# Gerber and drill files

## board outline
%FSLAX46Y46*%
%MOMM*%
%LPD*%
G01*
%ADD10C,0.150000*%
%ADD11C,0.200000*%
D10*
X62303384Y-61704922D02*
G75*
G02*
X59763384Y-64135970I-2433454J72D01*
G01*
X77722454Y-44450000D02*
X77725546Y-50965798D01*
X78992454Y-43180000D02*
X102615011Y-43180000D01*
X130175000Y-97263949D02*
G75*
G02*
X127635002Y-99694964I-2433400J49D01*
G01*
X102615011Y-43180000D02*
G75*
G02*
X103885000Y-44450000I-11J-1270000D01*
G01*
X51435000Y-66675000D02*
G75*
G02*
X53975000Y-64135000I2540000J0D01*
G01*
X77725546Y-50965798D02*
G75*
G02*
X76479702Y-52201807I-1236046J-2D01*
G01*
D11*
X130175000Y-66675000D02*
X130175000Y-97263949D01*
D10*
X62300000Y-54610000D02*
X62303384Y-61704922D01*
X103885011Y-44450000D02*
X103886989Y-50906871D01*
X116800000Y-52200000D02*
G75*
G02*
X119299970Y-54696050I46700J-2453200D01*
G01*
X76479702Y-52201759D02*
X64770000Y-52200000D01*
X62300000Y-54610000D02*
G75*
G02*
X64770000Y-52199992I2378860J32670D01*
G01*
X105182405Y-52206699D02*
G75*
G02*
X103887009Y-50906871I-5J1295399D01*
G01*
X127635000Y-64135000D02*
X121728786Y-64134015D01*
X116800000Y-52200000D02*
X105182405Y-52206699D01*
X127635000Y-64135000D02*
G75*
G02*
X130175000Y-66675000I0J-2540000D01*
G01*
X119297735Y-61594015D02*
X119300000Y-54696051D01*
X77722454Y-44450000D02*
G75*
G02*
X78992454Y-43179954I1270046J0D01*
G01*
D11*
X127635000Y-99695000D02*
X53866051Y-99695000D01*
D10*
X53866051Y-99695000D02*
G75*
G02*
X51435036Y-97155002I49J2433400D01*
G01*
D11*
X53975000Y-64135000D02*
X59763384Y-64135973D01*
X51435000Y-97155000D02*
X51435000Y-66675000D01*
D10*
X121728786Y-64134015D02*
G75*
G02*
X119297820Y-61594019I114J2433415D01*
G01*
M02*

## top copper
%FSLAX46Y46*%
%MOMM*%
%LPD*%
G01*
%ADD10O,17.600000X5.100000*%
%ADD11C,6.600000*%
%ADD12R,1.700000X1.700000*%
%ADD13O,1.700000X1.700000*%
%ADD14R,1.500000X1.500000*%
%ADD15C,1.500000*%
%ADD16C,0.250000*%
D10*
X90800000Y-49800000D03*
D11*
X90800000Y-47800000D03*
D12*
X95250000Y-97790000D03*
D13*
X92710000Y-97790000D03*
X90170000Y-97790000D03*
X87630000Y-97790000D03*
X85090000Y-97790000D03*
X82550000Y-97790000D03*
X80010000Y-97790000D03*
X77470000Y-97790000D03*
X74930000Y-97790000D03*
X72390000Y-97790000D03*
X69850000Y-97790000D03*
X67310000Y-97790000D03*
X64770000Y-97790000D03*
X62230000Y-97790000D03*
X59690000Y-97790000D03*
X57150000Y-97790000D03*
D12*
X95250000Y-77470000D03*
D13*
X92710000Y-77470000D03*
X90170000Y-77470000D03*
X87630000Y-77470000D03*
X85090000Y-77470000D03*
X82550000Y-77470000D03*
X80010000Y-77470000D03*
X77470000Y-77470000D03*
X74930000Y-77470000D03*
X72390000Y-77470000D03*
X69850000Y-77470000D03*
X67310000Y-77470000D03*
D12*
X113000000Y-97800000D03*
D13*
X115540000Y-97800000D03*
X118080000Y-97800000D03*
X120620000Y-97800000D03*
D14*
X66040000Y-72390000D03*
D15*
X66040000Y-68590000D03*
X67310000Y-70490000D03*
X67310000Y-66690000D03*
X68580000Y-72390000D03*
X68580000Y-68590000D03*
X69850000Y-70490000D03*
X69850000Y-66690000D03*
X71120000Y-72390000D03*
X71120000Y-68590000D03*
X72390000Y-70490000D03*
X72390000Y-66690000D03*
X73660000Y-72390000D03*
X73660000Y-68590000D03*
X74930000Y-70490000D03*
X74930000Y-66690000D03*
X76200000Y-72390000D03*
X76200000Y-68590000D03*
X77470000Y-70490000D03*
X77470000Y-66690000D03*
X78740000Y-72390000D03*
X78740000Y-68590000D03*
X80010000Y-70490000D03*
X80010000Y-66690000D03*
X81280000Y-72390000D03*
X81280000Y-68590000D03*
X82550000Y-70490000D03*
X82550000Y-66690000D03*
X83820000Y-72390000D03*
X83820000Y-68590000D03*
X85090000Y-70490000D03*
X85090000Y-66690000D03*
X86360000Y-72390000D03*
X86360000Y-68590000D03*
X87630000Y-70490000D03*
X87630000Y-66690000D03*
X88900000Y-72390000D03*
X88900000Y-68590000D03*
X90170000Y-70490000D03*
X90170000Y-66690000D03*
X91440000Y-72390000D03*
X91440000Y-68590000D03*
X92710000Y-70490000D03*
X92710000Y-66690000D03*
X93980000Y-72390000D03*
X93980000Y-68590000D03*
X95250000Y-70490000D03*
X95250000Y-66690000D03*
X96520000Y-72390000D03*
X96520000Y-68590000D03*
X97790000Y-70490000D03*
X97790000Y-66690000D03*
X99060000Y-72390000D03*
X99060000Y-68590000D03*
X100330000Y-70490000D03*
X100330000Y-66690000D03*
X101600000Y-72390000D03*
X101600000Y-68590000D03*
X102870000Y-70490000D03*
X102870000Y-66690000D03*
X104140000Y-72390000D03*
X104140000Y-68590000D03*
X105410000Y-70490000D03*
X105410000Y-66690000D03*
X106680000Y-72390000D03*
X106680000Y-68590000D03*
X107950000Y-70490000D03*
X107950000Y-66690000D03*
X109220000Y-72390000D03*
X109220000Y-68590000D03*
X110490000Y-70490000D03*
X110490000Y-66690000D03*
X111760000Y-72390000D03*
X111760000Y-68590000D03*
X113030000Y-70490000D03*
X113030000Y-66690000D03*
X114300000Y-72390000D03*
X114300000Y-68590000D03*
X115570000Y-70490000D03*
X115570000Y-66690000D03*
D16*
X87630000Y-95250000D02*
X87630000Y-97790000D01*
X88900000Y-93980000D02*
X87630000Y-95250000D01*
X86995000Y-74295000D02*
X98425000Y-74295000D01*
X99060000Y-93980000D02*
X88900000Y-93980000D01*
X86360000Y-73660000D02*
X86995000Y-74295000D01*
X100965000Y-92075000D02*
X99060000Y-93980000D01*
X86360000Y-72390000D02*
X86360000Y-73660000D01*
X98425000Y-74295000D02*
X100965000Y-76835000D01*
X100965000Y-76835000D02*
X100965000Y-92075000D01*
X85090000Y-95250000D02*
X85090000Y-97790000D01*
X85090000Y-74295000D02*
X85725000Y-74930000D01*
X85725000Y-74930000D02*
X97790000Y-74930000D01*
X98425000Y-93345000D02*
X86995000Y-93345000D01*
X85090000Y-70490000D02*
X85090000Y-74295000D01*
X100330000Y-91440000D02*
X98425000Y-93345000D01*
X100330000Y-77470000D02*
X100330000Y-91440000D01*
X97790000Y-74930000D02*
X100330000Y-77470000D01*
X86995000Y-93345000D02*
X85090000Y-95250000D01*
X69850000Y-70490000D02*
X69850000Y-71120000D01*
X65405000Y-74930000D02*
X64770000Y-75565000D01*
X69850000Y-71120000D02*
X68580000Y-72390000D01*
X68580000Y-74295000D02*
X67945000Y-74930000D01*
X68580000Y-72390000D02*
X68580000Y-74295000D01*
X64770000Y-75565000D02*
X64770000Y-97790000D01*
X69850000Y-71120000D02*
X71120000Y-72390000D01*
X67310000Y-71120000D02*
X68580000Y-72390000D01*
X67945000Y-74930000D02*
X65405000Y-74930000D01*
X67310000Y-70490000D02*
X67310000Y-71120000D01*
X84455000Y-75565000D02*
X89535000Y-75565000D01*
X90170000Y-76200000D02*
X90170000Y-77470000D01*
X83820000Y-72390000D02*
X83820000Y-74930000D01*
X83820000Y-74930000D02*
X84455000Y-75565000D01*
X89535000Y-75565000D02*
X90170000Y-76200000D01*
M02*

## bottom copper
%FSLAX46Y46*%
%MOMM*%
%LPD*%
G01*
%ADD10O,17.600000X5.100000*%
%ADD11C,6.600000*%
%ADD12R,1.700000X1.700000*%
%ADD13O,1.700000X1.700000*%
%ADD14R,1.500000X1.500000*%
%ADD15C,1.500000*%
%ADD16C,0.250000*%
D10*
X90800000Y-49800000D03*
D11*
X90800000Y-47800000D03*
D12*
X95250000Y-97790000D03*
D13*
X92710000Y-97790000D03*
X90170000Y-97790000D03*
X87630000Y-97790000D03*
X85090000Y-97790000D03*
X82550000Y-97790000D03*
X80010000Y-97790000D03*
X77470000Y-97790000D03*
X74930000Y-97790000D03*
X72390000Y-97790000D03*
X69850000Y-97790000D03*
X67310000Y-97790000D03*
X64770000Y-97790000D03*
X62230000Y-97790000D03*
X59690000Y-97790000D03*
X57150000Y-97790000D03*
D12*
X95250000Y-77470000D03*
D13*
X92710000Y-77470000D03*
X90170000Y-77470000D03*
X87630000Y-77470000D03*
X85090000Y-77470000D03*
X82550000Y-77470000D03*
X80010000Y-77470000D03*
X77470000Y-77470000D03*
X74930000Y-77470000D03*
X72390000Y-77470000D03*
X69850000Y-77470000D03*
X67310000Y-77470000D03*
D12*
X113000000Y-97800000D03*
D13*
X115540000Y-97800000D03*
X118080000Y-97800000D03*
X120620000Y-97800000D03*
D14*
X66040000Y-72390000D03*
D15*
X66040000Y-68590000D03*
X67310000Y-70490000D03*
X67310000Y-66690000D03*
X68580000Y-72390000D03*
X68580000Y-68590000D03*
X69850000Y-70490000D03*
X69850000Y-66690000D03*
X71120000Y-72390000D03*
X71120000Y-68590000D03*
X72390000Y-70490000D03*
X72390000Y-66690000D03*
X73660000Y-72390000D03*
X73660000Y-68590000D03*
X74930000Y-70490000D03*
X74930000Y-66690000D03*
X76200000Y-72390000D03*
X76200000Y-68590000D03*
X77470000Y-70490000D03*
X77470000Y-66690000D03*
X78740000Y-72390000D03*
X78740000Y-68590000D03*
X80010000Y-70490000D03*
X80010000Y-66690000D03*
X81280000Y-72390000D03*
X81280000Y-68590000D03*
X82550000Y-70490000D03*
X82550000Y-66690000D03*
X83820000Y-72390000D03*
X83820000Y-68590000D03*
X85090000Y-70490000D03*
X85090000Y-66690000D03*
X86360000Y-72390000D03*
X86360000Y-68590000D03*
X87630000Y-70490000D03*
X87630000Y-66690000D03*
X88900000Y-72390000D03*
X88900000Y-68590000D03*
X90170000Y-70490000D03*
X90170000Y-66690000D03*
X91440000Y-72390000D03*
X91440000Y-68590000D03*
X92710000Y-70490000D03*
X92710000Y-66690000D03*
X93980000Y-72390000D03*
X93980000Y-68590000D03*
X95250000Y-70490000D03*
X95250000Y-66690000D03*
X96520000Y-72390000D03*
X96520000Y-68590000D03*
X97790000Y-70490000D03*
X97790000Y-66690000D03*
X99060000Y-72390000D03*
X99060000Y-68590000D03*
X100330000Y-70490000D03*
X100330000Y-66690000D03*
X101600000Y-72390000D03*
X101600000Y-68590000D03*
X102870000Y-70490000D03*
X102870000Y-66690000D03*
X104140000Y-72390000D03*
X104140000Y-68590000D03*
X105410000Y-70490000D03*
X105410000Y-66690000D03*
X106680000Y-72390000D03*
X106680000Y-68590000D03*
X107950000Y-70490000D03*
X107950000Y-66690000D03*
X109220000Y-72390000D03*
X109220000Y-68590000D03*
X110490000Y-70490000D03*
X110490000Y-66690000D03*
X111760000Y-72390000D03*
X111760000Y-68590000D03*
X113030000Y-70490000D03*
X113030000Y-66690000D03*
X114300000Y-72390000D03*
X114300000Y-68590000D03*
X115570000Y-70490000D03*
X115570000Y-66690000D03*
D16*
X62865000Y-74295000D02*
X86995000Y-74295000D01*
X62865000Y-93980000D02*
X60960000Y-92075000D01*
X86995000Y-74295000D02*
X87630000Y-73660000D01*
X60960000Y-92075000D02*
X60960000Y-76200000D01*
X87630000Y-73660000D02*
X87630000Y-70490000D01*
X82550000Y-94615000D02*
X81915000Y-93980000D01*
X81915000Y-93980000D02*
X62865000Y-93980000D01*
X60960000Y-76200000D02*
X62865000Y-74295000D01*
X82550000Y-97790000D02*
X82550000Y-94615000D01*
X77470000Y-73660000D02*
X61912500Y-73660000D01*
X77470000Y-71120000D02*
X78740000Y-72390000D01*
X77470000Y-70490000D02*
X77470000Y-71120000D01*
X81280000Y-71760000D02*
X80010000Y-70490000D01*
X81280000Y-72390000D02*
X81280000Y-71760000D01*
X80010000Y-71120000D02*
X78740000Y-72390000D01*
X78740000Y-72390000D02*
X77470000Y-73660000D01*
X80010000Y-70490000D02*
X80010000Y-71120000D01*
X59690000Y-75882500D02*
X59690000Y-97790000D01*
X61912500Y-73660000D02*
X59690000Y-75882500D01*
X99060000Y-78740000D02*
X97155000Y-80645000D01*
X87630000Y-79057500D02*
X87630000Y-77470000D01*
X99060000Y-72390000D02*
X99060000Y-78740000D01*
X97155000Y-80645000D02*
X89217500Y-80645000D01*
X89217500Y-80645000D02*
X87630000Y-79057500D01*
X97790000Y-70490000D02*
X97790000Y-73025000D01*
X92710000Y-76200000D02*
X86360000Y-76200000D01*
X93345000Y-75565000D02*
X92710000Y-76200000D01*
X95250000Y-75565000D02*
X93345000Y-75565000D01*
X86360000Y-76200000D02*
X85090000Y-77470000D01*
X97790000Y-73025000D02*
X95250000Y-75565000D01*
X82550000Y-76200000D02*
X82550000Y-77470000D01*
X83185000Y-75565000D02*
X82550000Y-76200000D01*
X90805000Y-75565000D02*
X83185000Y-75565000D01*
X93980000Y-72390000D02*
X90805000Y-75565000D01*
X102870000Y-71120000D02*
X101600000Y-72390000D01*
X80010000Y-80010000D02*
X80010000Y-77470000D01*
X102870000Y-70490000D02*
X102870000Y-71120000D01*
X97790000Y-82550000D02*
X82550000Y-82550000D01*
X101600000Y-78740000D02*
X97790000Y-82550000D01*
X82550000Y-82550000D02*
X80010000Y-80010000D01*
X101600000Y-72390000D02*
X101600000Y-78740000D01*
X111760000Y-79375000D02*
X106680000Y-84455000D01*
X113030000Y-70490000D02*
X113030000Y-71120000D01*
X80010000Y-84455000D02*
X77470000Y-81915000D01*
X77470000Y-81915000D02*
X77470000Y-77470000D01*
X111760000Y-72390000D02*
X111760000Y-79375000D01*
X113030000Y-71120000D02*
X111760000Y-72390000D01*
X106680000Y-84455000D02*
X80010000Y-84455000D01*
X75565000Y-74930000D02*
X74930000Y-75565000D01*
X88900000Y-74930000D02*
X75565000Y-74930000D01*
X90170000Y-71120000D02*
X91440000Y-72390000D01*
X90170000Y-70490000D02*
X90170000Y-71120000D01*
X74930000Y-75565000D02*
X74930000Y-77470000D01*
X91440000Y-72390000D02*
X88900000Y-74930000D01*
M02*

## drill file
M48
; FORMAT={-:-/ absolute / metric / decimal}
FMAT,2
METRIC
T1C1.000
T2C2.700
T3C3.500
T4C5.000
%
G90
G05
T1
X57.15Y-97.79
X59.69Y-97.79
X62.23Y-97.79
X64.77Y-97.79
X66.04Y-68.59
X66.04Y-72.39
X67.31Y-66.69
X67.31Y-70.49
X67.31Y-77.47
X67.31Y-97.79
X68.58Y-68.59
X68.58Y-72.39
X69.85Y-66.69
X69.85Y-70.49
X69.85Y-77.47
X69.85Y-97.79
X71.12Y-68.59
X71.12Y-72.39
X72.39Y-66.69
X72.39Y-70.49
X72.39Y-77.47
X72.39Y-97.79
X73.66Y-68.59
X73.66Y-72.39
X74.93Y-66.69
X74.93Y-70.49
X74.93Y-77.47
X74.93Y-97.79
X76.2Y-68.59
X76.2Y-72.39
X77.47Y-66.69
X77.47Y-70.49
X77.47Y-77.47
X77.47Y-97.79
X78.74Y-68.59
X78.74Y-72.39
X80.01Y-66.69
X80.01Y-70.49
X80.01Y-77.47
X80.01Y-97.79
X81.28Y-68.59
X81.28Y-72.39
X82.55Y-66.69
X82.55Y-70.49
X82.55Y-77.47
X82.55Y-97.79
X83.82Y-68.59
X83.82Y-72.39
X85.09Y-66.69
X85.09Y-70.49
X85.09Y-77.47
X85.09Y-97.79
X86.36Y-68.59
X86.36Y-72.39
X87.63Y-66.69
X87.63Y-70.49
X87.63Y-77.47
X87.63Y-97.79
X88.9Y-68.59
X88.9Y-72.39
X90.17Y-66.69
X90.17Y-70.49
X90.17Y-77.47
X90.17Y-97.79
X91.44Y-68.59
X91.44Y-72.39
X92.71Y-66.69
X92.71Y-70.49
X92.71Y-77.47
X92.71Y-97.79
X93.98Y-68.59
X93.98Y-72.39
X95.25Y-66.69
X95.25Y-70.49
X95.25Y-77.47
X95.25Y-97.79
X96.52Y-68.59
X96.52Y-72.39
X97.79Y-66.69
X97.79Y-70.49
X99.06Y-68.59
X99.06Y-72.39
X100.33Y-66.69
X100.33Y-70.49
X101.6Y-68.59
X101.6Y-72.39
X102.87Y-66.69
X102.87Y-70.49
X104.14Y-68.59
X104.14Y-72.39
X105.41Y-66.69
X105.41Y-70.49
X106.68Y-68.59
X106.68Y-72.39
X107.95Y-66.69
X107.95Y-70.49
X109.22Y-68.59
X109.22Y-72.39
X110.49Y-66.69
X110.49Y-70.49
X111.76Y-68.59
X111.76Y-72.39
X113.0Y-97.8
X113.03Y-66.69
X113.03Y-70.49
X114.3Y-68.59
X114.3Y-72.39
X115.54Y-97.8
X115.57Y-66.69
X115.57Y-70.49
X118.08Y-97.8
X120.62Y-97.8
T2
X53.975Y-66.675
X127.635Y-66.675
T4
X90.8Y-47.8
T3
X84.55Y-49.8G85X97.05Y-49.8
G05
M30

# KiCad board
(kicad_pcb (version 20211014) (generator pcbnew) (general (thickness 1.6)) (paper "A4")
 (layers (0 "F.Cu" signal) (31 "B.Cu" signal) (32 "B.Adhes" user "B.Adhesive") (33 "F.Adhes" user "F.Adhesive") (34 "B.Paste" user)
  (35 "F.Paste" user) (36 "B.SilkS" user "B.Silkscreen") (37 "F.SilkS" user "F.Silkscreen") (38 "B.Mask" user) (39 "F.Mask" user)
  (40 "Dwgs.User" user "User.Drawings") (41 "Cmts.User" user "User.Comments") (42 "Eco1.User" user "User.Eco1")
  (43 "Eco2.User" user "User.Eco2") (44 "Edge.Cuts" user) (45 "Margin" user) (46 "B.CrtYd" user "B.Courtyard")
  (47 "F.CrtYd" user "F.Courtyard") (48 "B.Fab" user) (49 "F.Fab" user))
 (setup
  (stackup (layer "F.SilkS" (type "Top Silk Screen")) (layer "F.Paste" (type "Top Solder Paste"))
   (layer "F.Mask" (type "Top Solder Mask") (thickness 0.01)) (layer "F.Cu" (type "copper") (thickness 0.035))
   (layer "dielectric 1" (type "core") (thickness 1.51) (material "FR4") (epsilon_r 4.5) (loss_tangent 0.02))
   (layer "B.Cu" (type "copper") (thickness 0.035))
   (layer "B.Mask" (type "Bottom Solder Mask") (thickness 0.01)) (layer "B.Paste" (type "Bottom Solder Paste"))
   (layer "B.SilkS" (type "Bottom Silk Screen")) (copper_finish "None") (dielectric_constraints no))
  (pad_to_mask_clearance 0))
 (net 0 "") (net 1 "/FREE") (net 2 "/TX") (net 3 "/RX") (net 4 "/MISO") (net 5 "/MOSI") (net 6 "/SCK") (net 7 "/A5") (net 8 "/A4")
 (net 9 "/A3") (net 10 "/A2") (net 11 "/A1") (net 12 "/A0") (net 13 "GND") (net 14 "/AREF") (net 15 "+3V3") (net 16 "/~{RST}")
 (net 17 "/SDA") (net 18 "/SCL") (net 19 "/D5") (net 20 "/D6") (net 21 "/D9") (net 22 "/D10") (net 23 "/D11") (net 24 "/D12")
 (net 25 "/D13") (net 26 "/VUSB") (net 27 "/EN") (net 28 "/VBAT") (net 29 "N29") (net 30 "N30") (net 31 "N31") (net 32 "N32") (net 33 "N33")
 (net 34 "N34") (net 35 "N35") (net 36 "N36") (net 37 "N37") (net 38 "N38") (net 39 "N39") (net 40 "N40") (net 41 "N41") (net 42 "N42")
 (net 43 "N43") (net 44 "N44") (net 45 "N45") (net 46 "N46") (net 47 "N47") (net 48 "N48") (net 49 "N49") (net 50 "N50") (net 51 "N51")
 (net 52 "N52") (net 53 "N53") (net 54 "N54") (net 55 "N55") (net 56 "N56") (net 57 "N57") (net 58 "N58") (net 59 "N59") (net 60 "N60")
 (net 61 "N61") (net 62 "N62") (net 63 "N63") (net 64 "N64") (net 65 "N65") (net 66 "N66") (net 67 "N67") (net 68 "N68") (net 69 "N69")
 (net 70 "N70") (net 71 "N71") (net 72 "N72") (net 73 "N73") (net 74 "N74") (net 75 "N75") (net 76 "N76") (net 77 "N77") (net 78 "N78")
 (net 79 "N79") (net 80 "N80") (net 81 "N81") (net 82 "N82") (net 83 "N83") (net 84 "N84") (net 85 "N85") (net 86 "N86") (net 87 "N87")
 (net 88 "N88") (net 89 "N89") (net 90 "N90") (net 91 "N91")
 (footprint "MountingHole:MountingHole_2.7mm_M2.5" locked (layer "F.Cu") (at 53.975 66.675)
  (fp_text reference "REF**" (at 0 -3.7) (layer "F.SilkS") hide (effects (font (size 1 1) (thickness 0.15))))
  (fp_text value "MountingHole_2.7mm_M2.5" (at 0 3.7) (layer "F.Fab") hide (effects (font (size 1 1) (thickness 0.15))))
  (pad "" np_thru_hole circle locked (at 0 0) (size 2.7 2.7) (drill 2.7) (layers *.Cu *.Mask)))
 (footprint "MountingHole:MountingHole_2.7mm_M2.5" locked (layer "F.Cu") (at 127.635 66.675)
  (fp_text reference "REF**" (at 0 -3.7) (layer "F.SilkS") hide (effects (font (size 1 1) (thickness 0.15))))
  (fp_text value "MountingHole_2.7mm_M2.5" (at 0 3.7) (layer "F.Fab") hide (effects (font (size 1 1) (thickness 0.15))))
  (pad "" np_thru_hole circle locked (at 0 0) (size 2.7 2.7) (drill 2.7) (layers *.Cu *.Mask)))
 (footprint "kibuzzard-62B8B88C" (layer "F.Cu") (at 90.8 58.674)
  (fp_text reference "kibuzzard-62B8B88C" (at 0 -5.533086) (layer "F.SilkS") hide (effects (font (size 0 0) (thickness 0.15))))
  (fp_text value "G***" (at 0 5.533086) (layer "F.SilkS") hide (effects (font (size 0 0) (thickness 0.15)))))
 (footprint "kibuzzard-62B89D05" (layer "F.Cu") (at 125.9 97.8)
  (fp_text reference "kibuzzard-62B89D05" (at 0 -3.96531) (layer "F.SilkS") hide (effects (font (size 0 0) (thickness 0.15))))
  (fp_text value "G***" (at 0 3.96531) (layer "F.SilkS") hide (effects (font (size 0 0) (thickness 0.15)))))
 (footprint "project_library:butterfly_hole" (layer "F.Cu") (at 90.8 49.8)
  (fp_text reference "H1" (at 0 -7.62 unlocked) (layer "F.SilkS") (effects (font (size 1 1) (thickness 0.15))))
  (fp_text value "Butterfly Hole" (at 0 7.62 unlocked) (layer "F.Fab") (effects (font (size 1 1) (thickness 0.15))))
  (pad "" np_thru_hole oval (at 0 0) (size 17.6 5.1) (drill oval 16 3.5) (layers F&B.Cu *.Mask))
  (pad "" np_thru_hole circle (at 0 -2) (size 6.6 6.6) (drill 5) (layers F&B.Cu *.Mask)))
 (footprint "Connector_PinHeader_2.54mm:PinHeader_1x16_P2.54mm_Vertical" (layer "B.Cu") (at 95.25 97.79 90)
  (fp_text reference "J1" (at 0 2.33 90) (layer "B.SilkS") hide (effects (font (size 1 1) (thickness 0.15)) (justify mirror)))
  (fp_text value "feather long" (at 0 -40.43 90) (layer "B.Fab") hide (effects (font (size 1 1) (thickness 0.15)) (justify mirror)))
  (pad "1" thru_hole rect locked (at 0 0 90) (size 1.7 1.7) (drill 1) (layers *.Cu *.Mask) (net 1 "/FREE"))
  (pad "2" thru_hole oval locked (at 0 -2.54 90) (size 1.7 1.7) (drill 1) (layers *.Cu *.Mask) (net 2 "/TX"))
  (pad "3" thru_hole oval locked (at 0 -5.08 90) (size 1.7 1.7) (drill 1) (layers *.Cu *.Mask) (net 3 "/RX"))
  (pad "4" thru_hole oval locked (at 0 -7.62 90) (size 1.7 1.7) (drill 1) (layers *.Cu *.Mask) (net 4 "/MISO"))
  (pad "5" thru_hole oval locked (at 0 -10.16 90) (size 1.7 1.7) (drill 1) (layers *.Cu *.Mask) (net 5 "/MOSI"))
  (pad "6" thru_hole oval locked (at 0 -12.7 90) (size 1.7 1.7) (drill 1) (layers *.Cu *.Mask) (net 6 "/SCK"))
  (pad "7" thru_hole oval locked (at 0 -15.24 90) (size 1.7 1.7) (drill 1) (layers *.Cu *.Mask) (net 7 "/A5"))
  (pad "8" thru_hole oval locked (at 0 -17.78 90) (size 1.7 1.7) (drill 1) (layers *.Cu *.Mask) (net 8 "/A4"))
  (pad "9" thru_hole oval locked (at 0 -20.32 90) (size 1.7 1.7) (drill 1) (layers *.Cu *.Mask) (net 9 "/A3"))
  (pad "10" thru_hole oval locked (at 0 -22.86 90) (size 1.7 1.7) (drill 1) (layers *.Cu *.Mask) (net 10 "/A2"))
  (pad "11" thru_hole oval locked (at 0 -25.4 90) (size 1.7 1.7) (drill 1) (layers *.Cu *.Mask) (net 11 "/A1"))
  (pad "12" thru_hole oval locked (at 0 -27.94 90) (size 1.7 1.7) (drill 1) (layers *.Cu *.Mask) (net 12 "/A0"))
  (pad "13" thru_hole oval locked (at 0 -30.48 90) (size 1.7 1.7) (drill 1) (layers *.Cu *.Mask) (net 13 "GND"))
  (pad "14" thru_hole oval locked (at 0 -33.02 90) (size 1.7 1.7) (drill 1) (layers *.Cu *.Mask) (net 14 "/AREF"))
  (pad "15" thru_hole oval locked (at 0 -35.56 90) (size 1.7 1.7) (drill 1) (layers *.Cu *.Mask) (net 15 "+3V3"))
  (pad "16" thru_hole oval locked (at 0 -38.1 90) (size 1.7 1.7) (drill 1) (layers *.Cu *.Mask) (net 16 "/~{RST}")))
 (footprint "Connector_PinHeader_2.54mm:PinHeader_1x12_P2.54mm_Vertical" (layer "B.Cu") (at 95.25 77.47 90)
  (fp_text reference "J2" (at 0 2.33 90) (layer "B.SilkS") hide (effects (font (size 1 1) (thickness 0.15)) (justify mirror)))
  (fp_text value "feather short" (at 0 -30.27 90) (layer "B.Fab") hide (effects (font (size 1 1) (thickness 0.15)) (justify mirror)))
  (pad "1" thru_hole rect locked (at 0 0 90) (size 1.7 1.7) (drill 1) (layers *.Cu *.Mask) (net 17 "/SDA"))
  (pad "2" thru_hole oval locked (at 0 -2.54 90) (size 1.7 1.7) (drill 1) (layers *.Cu *.Mask) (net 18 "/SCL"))
  (pad "3" thru_hole oval locked (at 0 -5.08 90) (size 1.7 1.7) (drill 1) (layers *.Cu *.Mask) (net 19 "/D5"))
  (pad "4" thru_hole oval locked (at 0 -7.62 90) (size 1.7 1.7) (drill 1) (layers *.Cu *.Mask) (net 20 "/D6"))
  (pad "5" thru_hole oval locked (at 0 -10.16 90) (size 1.7 1.7) (drill 1) (layers *.Cu *.Mask) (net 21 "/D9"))
  (pad "6" thru_hole oval locked (at 0 -12.7 90) (size 1.7 1.7) (drill 1) (layers *.Cu *.Mask) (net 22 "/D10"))
  (pad "7" thru_hole oval locked (at 0 -15.24 90) (size 1.7 1.7) (drill 1) (layers *.Cu *.Mask) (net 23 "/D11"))
  (pad "8" thru_hole oval locked (at 0 -17.78 90) (size 1.7 1.7) (drill 1) (layers *.Cu *.Mask) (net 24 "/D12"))
  (pad "9" thru_hole oval locked (at 0 -20.32 90) (size 1.7 1.7) (drill 1) (layers *.Cu *.Mask) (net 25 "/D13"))
  (pad "10" thru_hole oval locked (at 0 -22.86 90) (size 1.7 1.7) (drill 1) (layers *.Cu *.Mask) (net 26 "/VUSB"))
  (pad "11" thru_hole oval locked (at 0 -25.4 90) (size 1.7 1.7) (drill 1) (layers *.Cu *.Mask) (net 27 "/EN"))
  (pad "12" thru_hole oval locked (at 0 -27.94 90) (size 1.7 1.7) (drill 1) (layers *.Cu *.Mask) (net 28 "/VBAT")))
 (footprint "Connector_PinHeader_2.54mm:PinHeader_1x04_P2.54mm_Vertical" (layer "B.Cu") (at 113 97.8 -90)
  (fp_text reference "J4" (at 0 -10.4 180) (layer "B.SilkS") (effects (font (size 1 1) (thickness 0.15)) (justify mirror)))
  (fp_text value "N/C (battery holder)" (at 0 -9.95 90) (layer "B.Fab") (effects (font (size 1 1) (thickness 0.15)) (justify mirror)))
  (pad "1" thru_hole rect (at 0 0 270) (size 1.7 1.7) (drill 1) (layers *.Cu *.Mask) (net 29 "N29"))
  (pad "2" thru_hole oval (at 0 -2.54 270) (size 1.7 1.7) (drill 1) (layers *.Cu *.Mask) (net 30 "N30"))
  (pad "3" thru_hole oval (at 0 -5.08 270) (size 1.7 1.7) (drill 1) (layers *.Cu *.Mask) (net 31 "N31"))
  (pad "4" thru_hole oval (at 0 -7.62 270) (size 1.7 1.7) (drill 1) (layers *.Cu *.Mask) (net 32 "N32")))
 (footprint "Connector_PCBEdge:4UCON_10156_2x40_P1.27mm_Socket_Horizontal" (layer "B.Cu") (at 66.04 72.39)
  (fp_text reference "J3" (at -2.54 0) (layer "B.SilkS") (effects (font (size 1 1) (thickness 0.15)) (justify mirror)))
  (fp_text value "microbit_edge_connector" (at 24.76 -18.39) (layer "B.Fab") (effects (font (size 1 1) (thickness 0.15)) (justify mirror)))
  (pad "1" thru_hole rect (at 0 0) (size 1.5 1.5) (drill 1) (layers *.Cu *.Mask) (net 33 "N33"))
  (pad "2" thru_hole circle (at 0 -3.8) (size 1.5 1.5) (drill 1) (layers *.Cu *.Mask) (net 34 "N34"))
  (pad "3" thru_hole circle (at 1.27 -1.9) (size 1.5 1.5) (drill 1) (layers *.Cu *.Mask) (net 13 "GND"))
  (pad "4" thru_hole circle (at 1.27 -5.7) (size 1.5 1.5) (drill 1) (layers *.Cu *.Mask) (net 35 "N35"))
  (pad "5" thru_hole circle (at 2.54 0) (size 1.5 1.5) (drill 1) (layers *.Cu *.Mask) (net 13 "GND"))
  (pad "6" thru_hole circle (at 2.54 -3.8) (size 1.5 1.5) (drill 1) (layers *.Cu *.Mask) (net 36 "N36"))
  (pad "7" thru_hole circle (at 3.81 -1.9) (size 1.5 1.5) (drill 1) (layers *.Cu *.Mask) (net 13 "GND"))
  (pad "8" thru_hole circle (at 3.81 -5.7) (size 1.5 1.5) (drill 1) (layers *.Cu *.Mask) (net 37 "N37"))
  (pad "9" thru_hole circle (at 5.08 0) (size 1.5 1.5) (drill 1) (layers *.Cu *.Mask) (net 13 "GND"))
  (pad "10" thru_hole circle (at 5.08 -3.8) (size 1.5 1.5) (drill 1) (layers *.Cu *.Mask) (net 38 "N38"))
  (pad "11" thru_hole circle (at 6.35 -1.9) (size 1.5 1.5) (drill 1) (layers *.Cu *.Mask) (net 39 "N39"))
  (pad "12" thru_hole circle (at 6.35 -5.7) (size 1.5 1.5) (drill 1) (layers *.Cu *.Mask) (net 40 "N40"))
  (pad "13" thru_hole circle (at 7.62 0) (size 1.5 1.5) (drill 1) (layers *.Cu *.Mask) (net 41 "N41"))
  (pad "14" thru_hole circle (at 7.62 -3.8) (size 1.5 1.5) (drill 1) (layers *.Cu *.Mask) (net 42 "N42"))
  (pad "15" thru_hole circle (at 8.89 -1.9) (size 1.5 1.5) (drill 1) (layers *.Cu *.Mask) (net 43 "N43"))
  (pad "16" thru_hole circle (at 8.89 -5.7) (size 1.5 1.5) (drill 1) (layers *.Cu *.Mask) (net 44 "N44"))
  (pad "17" thru_hole circle (at 10.16 0) (size 1.5 1.5) (drill 1) (layers *.Cu *.Mask) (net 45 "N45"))
  (pad "18" thru_hole circle (at 10.16 -3.8) (size 1.5 1.5) (drill 1) (layers *.Cu *.Mask) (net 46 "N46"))
  (pad "19" thru_hole circle (at 11.43 -1.9) (size 1.5 1.5) (drill 1) (layers *.Cu *.Mask) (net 15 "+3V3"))
  (pad "20" thru_hole circle (at 11.43 -5.7) (size 1.5 1.5) (drill 1) (layers *.Cu *.Mask) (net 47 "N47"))
  (pad "21" thru_hole circle (at 12.7 0) (size 1.5 1.5) (drill 1) (layers *.Cu *.Mask) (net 15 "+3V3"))
  (pad "22" thru_hole circle (at 12.7 -3.8) (size 1.5 1.5) (drill 1) (layers *.Cu *.Mask) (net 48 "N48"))
  (pad "23" thru_hole circle (at 13.97 -1.9) (size 1.5 1.5) (drill 1) (layers *.Cu *.Mask) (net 15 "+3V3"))
  (pad "24" thru_hole circle (at 13.97 -5.7) (size 1.5 1.5) (drill 1) (layers *.Cu *.Mask) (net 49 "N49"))
  (pad "25" thru_hole circle (at 15.24 0) (size 1.5 1.5) (drill 1) (layers *.Cu *.Mask) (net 15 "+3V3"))
  (pad "26" thru_hole circle (at 15.24 -3.8) (size 1.5 1.5) (drill 1) (layers *.Cu *.Mask) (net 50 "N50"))
  (pad "27" thru_hole circle (at 16.51 -1.9) (size 1.5 1.5) (drill 1) (layers *.Cu *.Mask) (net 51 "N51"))
  (pad "28" thru_hole circle (at 16.51 -5.7) (size 1.5 1.5) (drill 1) (layers *.Cu *.Mask) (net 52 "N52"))
  (pad "29" thru_hole circle (at 17.78 0) (size 1.5 1.5) (drill 1) (layers *.Cu *.Mask) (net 19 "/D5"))
  (pad "30" thru_hole circle (at 17.78 -3.8) (size 1.5 1.5) (drill 1) (layers *.Cu *.Mask) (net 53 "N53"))
  (pad "31" thru_hole circle (at 19.05 -1.9) (size 1.5 1.5) (drill 1) (layers *.Cu *.Mask) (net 5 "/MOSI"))
  (pad "32" thru_hole circle (at 19.05 -5.7) (size 1.5 1.5) (drill 1) (layers *.Cu *.Mask) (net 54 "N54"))
  (pad "33" thru_hole circle (at 20.32 0) (size 1.5 1.5) (drill 1) (layers *.Cu *.Mask) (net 4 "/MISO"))
  (pad "34" thru_hole circle (at 20.32 -3.8) (size 1.5 1.5) (drill 1) (layers *.Cu *.Mask) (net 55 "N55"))
  (pad "35" thru_hole circle (at 21.59 -1.9) (size 1.5 1.5) (drill 1) (layers *.Cu *.Mask) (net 6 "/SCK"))
  (pad "36" thru_hole circle (at 21.59 -5.7) (size 1.5 1.5) (drill 1) (layers *.Cu *.Mask) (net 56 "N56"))
  (pad "37" thru_hole circle (at 22.86 0) (size 1.5 1.5) (drill 1) (layers *.Cu *.Mask) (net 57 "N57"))
  (pad "38" thru_hole circle (at 22.86 -3.8) (size 1.5 1.5) (drill 1) (layers *.Cu *.Mask) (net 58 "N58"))
  (pad "39" thru_hole circle (at 24.13 -1.9) (size 1.5 1.5) (drill 1) (layers *.Cu *.Mask) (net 25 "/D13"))
  (pad "40" thru_hole circle (at 24.13 -5.7) (size 1.5 1.5) (drill 1) (layers *.Cu *.Mask) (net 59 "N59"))
  (pad "41" thru_hole circle (at 25.4 0) (size 1.5 1.5) (drill 1) (layers *.Cu *.Mask) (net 25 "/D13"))
  (pad "42" thru_hole circle (at 25.4 -3.8) (size 1.5 1.5) (drill 1) (layers *.Cu *.Mask) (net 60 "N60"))
  (pad "43" thru_hole circle (at 26.67 -1.9) (size 1.5 1.5) (drill 1) (layers *.Cu *.Mask) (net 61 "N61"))
  (pad "44" thru_hole circle (at 26.67 -5.7) (size 1.5 1.5) (drill 1) (layers *.Cu *.Mask) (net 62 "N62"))
  (pad "45" thru_hole circle (at 27.94 0) (size 1.5 1.5) (drill 1) (layers *.Cu *.Mask) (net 22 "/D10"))
  (pad "46" thru_hole circle (at 27.94 -3.8) (size 1.5 1.5) (drill 1) (layers *.Cu *.Mask) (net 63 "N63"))
  (pad "47" thru_hole circle (at 29.21 -1.9) (size 1.5 1.5) (drill 1) (layers *.Cu *.Mask) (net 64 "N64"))
  (pad "48" thru_hole circle (at 29.21 -5.7) (size 1.5 1.5) (drill 1) (layers *.Cu *.Mask) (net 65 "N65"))
  (pad "49" thru_hole circle (at 30.48 0) (size 1.5 1.5) (drill 1) (layers *.Cu *.Mask) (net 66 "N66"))
  (pad "50" thru_hole circle (at 30.48 -3.8) (size 1.5 1.5) (drill 1) (layers *.Cu *.Mask) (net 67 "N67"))
  (pad "51" thru_hole circle (at 31.75 -1.9) (size 1.5 1.5) (drill 1) (layers *.Cu *.Mask) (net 21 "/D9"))
  (pad "52" thru_hole circle (at 31.75 -5.7) (size 1.5 1.5) (drill 1) (layers *.Cu *.Mask) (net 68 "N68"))
  (pad "53" thru_hole circle (at 33.02 0) (size 1.5 1.5) (drill 1) (layers *.Cu *.Mask) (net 20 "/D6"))
  (pad "54" thru_hole circle (at 33.02 -3.8) (size 1.5 1.5) (drill 1) (layers *.Cu *.Mask) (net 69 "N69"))
  (pad "55" thru_hole circle (at 34.29 -1.9) (size 1.5 1.5) (drill 1) (layers *.Cu *.Mask) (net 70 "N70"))
  (pad "56" thru_hole circle (at 34.29 -5.7) (size 1.5 1.5) (drill 1) (layers *.Cu *.Mask) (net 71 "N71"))
  (pad "57" thru_hole circle (at 35.56 0) (size 1.5 1.5) (drill 1) (layers *.Cu *.Mask) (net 23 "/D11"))
  (pad "58" thru_hole circle (at 35.56 -3.8) (size 1.5 1.5) (drill 1) (layers *.Cu *.Mask) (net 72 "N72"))
  (pad "59" thru_hole circle (at 36.83 -1.9) (size 1.5 1.5) (drill 1) (layers *.Cu *.Mask) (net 23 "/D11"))
  (pad "60" thru_hole circle (at 36.83 -5.7) (size 1.5 1.5) (drill 1) (layers *.Cu *.Mask) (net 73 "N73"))
  (pad "61" thru_hole circle (at 38.1 0) (size 1.5 1.5) (drill 1) (layers *.Cu *.Mask) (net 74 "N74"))
  (pad "62" thru_hole circle (at 38.1 -3.8) (size 1.5 1.5) (drill 1) (layers *.Cu *.Mask) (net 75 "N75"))
  (pad "63" thru_hole circle (at 39.37 -1.9) (size 1.5 1.5) (drill 1) (layers *.Cu *.Mask) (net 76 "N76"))
  (pad "64" thru_hole circle (at 39.37 -5.7) (size 1.5 1.5) (drill 1) (layers *.Cu *.Mask) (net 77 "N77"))
  (pad "65" thru_hole circle (at 40.64 0) (size 1.5 1.5) (drill 1) (layers *.Cu *.Mask) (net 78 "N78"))
  (pad "66" thru_hole circle (at 40.64 -3.8) (size 1.5 1.5) (drill 1) (layers *.Cu *.Mask) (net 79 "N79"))
  (pad "67" thru_hole circle (at 41.91 -1.9) (size 1.5 1.5) (drill 1) (layers *.Cu *.Mask) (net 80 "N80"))
  (pad "68" thru_hole circle (at 41.91 -5.7) (size 1.5 1.5) (drill 1) (layers *.Cu *.Mask) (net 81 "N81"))
  (pad "69" thru_hole circle (at 43.18 0) (size 1.5 1.5) (drill 1) (layers *.Cu *.Mask) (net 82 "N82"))
  (pad "70" thru_hole circle (at 43.18 -3.8) (size 1.5 1.5) (drill 1) (layers *.Cu *.Mask) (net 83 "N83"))
  (pad "71" thru_hole circle (at 44.45 -1.9) (size 1.5 1.5) (drill 1) (layers *.Cu *.Mask) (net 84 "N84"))
  (pad "72" thru_hole circle (at 44.45 -5.7) (size 1.5 1.5) (drill 1) (layers *.Cu *.Mask) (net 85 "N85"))
  (pad "73" thru_hole circle (at 45.72 0) (size 1.5 1.5) (drill 1) (layers *.Cu *.Mask) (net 24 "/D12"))
  (pad "74" thru_hole circle (at 45.72 -3.8) (size 1.5 1.5) (drill 1) (layers *.Cu *.Mask) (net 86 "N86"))
  (pad "75" thru_hole circle (at 46.99 -1.9) (size 1.5 1.5) (drill 1) (layers *.Cu *.Mask) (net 24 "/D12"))
  (pad "76" thru_hole circle (at 46.99 -5.7) (size 1.5 1.5) (drill 1) (layers *.Cu *.Mask) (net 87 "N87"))
  (pad "77" thru_hole circle (at 48.26 0) (size 1.5 1.5) (drill 1) (layers *.Cu *.Mask) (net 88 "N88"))
  (pad "78" thru_hole circle (at 48.26 -3.8) (size 1.5 1.5) (drill 1) (layers *.Cu *.Mask) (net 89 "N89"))
  (pad "79" thru_hole circle (at 49.53 -1.9) (size 1.5 1.5) (drill 1) (layers *.Cu *.Mask) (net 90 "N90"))
  (pad "80" thru_hole circle (at 49.53 -5.7) (size 1.5 1.5) (drill 1) (layers *.Cu *.Mask) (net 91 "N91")))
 (gr_arc (start 62.303384 61.704922) (mid 61.552524 63.462854) (end 59.763384 64.135973) (layer "Edge.Cuts") (width 0.15))
 (gr_line (start 77.722454 44.45) (end 77.725546 50.965798) (layer "Edge.Cuts") (width 0.15))
 (gr_line (start 78.992454 43.18) (end 102.615011 43.18) (layer "Edge.Cuts") (width 0.15))
 (gr_arc (start 130.175 97.263949) (mid 129.424162 99.021903) (end 127.635 99.695) (layer "Edge.Cuts") (width 0.15))
 (gr_arc (start 102.615011 43.18) (mid 103.513037 43.551974) (end 103.885011 44.45) (layer "Edge.Cuts") (width 0.15))
 (gr_arc (start 51.435 66.675) (mid 52.178949 64.878949) (end 53.975 64.135) (layer "Edge.Cuts") (width 0.15))
 (gr_arc (start 77.725546 50.965798) (mid 77.360043 51.843255) (end 76.479702 52.201759) (layer "Edge.Cuts") (width 0.15))
 (gr_line (start 130.175 66.675) (end 130.175 97.263949) (layer "Edge.Cuts") (width 0.2))
 (gr_line (start 62.3 54.61) (end 62.303384 61.704922) (layer "Edge.Cuts") (width 0.15))
 (gr_line (start 103.885011 44.45) (end 103.886989 50.906871) (layer "Edge.Cuts") (width 0.15))
 (gr_arc (start 116.8 52.2) (mid 118.580337 52.916849) (end 119.3 54.696051) (layer "Edge.Cuts") (width 0.15))
 (gr_line (start 76.479702 52.201759) (end 64.77 52.2) (layer "Edge.Cuts") (width 0.15))
 (gr_arc (start 62.3 54.61) (mid 63.017402 52.874515) (end 64.77 52.2) (layer "Edge.Cuts") (width 0.15))
 (gr_arc (start 105.182405 52.206699) (mid 104.264847 51.82572) (end 103.886989 50.906871) (layer "Edge.Cuts") (width 0.15))
 (gr_line (start 127.635 64.135) (end 121.728786 64.134015) (layer "Edge.Cuts") (width 0.15))
 (gr_line (start 116.8 52.2) (end 105.182405 52.206699) (layer "Edge.Cuts") (width 0.15))
 (gr_arc (start 127.635 64.135) (mid 129.431051 64.878949) (end 130.175 66.675) (layer "Edge.Cuts") (width 0.15))
 (gr_line (start 119.297735 61.594015) (end 119.3 54.696051) (layer "Edge.Cuts") (width 0.15))
 (gr_arc (start 77.722454 44.45) (mid 78.094428 43.551974) (end 78.992454 43.18) (layer "Edge.Cuts") (width 0.15))
 (gr_line (start 127.635 99.695) (end 53.866051 99.695) (layer "Edge.Cuts") (width 0.2))
 (gr_arc (start 53.866051 99.695) (mid 52.108097 98.944162) (end 51.435 97.155) (layer "Edge.Cuts") (width 0.15))
 (gr_line (start 53.975 64.135) (end 59.763384 64.135973) (layer "Edge.Cuts") (width 0.2))
 (gr_line (start 51.435 97.155) (end 51.435 66.675) (layer "Edge.Cuts") (width 0.2))
 (gr_arc (start 121.728786 64.134015) (mid 119.970854 63.383155) (end 119.297735 61.594015) (layer "Edge.Cuts") (width 0.15))
 (segment (start 87.63 95.25) (end 87.63 97.79) (width 0.25) (layer "F.Cu") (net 4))
 (segment (start 88.9 93.98) (end 87.63 95.25) (width 0.25) (layer "F.Cu") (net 4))
 (segment (start 86.995 74.295) (end 98.425 74.295) (width 0.25) (layer "F.Cu") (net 4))
 (segment (start 99.06 93.98) (end 88.9 93.98) (width 0.25) (layer "F.Cu") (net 4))
 (segment (start 86.36 73.66) (end 86.995 74.295) (width 0.25) (layer "F.Cu") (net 4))
 (segment (start 100.965 92.075) (end 99.06 93.98) (width 0.25) (layer "F.Cu") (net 4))
 (segment (start 86.36 72.39) (end 86.36 73.66) (width 0.25) (layer "F.Cu") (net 4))
 (segment (start 98.425 74.295) (end 100.965 76.835) (width 0.25) (layer "F.Cu") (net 4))
 (segment (start 100.965 76.835) (end 100.965 92.075) (width 0.25) (layer "F.Cu") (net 4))
 (segment (start 85.09 95.25) (end 85.09 97.79) (width 0.25) (layer "F.Cu") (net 5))
 (segment (start 85.09 74.295) (end 85.725 74.93) (width 0.25) (layer "F.Cu") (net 5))
 (segment (start 85.725 74.93) (end 97.79 74.93) (width 0.25) (layer "F.Cu") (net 5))
 (segment (start 98.425 93.345) (end 86.995 93.345) (width 0.25) (layer "F.Cu") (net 5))
 (segment (start 85.09 70.49) (end 85.09 74.295) (width 0.25) (layer "F.Cu") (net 5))
 (segment (start 100.33 91.44) (end 98.425 93.345) (width 0.25) (layer "F.Cu") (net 5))
 (segment (start 100.33 77.47) (end 100.33 91.44) (width 0.25) (layer "F.Cu") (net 5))
 (segment (start 97.79 74.93) (end 100.33 77.47) (width 0.25) (layer "F.Cu") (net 5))
 (segment (start 86.995 93.345) (end 85.09 95.25) (width 0.25) (layer "F.Cu") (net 5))
 (segment (start 62.865 74.295) (end 86.995 74.295) (width 0.25) (layer "B.Cu") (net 6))
 (segment (start 62.865 93.98) (end 60.96 92.075) (width 0.25) (layer "B.Cu") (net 6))
 (segment (start 86.995 74.295) (end 87.63 73.66) (width 0.25) (layer "B.Cu") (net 6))
 (segment (start 60.96 92.075) (end 60.96 76.2) (width 0.25) (layer "B.Cu") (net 6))
 (segment (start 87.63 73.66) (end 87.63 70.49) (width 0.25) (layer "B.Cu") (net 6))
 (segment (start 82.55 94.615) (end 81.915 93.98) (width 0.25) (layer "B.Cu") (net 6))
 (segment (start 81.915 93.98) (end 62.865 93.98) (width 0.25) (layer "B.Cu") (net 6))
 (segment (start 60.96 76.2) (end 62.865 74.295) (width 0.25) (layer "B.Cu") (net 6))
 (segment (start 82.55 97.79) (end 82.55 94.615) (width 0.25) (layer "B.Cu") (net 6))
 (segment (start 69.85 70.49) (end 69.85 71.12) (width 0.25) (layer "F.Cu") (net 13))
 (segment (start 65.405 74.93) (end 64.77 75.565) (width 0.25) (layer "F.Cu") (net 13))
 (segment (start 69.85 71.12) (end 68.58 72.39) (width 0.25) (layer "F.Cu") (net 13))
 (segment (start 68.58 74.295) (end 67.945 74.93) (width 0.25) (layer "F.Cu") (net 13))
 (segment (start 68.58 72.39) (end 68.58 74.295) (width 0.25) (layer "F.Cu") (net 13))
 (segment (start 64.77 75.565) (end 64.77 97.79) (width 0.25) (layer "F.Cu") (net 13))
 (segment (start 69.85 71.12) (end 71.12 72.39) (width 0.25) (layer "F.Cu") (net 13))
 (segment (start 67.31 71.12) (end 68.58 72.39) (width 0.25) (layer "F.Cu") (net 13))
 (segment (start 67.945 74.93) (end 65.405 74.93) (width 0.25) (layer "F.Cu") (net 13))
 (segment (start 67.31 70.49) (end 67.31 71.12) (width 0.25) (layer "F.Cu") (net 13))
 (segment (start 77.47 73.66) (end 61.9125 73.66) (width 0.25) (layer "B.Cu") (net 15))
 (segment (start 77.47 71.12) (end 78.74 72.39) (width 0.25) (layer "B.Cu") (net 15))
 (segment (start 77.47 70.49) (end 77.47 71.12) (width 0.25) (layer "B.Cu") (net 15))
 (segment (start 81.28 71.76) (end 80.01 70.49) (width 0.25) (layer "B.Cu") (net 15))
 (segment (start 81.28 72.39) (end 81.28 71.76) (width 0.25) (layer "B.Cu") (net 15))
 (segment (start 80.01 71.12) (end 78.74 72.39) (width 0.25) (layer "B.Cu") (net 15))
 (segment (start 78.74 72.39) (end 77.47 73.66) (width 0.25) (layer "B.Cu") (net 15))
 (segment (start 80.01 70.49) (end 80.01 71.12) (width 0.25) (layer "B.Cu") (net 15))
 (segment (start 59.69 75.8825) (end 59.69 97.79) (width 0.25) (layer "B.Cu") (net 15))
 (segment (start 61.9125 73.66) (end 59.69 75.8825) (width 0.25) (layer "B.Cu") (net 15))
 (segment (start 84.455 75.565) (end 89.535 75.565) (width 0.25) (layer "F.Cu") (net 19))
 (segment (start 90.17 76.2) (end 90.17 77.47) (width 0.25) (layer "F.Cu") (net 19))
 (segment (start 83.82 72.39) (end 83.82 74.93) (width 0.25) (layer "F.Cu") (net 19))
 (segment (start 83.82 74.93) (end 84.455 75.565) (width 0.25) (layer "F.Cu") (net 19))
 (segment (start 89.535 75.565) (end 90.17 76.2) (width 0.25) (layer "F.Cu") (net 19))
 (segment (start 99.06 78.74) (end 97.155 80.645) (width 0.25) (layer "B.Cu") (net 20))
 (segment (start 87.63 79.0575) (end 87.63 77.47) (width 0.25) (layer "B.Cu") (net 20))
 (segment (start 99.06 72.39) (end 99.06 78.74) (width 0.25) (layer "B.Cu") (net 20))
 (segment (start 97.155 80.645) (end 89.2175 80.645) (width 0.25) (layer "B.Cu") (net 20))
 (segment (start 89.2175 80.645) (end 87.63 79.0575) (width 0.25) (layer "B.Cu") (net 20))
 (segment (start 97.79 70.49) (end 97.79 73.025) (width 0.25) (layer "B.Cu") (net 21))
 (segment (start 92.71 76.2) (end 86.36 76.2) (width 0.25) (layer "B.Cu") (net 21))
 (segment (start 93.345 75.565) (end 92.71 76.2) (width 0.25) (layer "B.Cu") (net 21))
 (segment (start 95.25 75.565) (end 93.345 75.565) (width 0.25) (layer "B.Cu") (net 21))
 (segment (start 86.36 76.2) (end 85.09 77.47) (width 0.25) (layer "B.Cu") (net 21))
 (segment (start 97.79 73.025) (end 95.25 75.565) (width 0.25) (layer "B.Cu") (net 21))
 (segment (start 82.55 76.2) (end 82.55 77.47) (width 0.25) (layer "B.Cu") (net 22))
 (segment (start 83.185 75.565) (end 82.55 76.2) (width 0.25) (layer "B.Cu") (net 22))
 (segment (start 90.805 75.565) (end 83.185 75.565) (width 0.25) (layer "B.Cu") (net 22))
 (segment (start 93.98 72.39) (end 90.805 75.565) (width 0.25) (layer "B.Cu") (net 22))
 (segment (start 102.87 71.12) (end 101.6 72.39) (width 0.25) (layer "B.Cu") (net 23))
 (segment (start 80.01 80.01) (end 80.01 77.47) (width 0.25) (layer "B.Cu") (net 23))
 (segment (start 102.87 70.49) (end 102.87 71.12) (width 0.25) (layer "B.Cu") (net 23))
 (segment (start 97.79 82.55) (end 82.55 82.55) (width 0.25) (layer "B.Cu") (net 23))
 (segment (start 101.6 78.74) (end 97.79 82.55) (width 0.25) (layer "B.Cu") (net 23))
 (segment (start 82.55 82.55) (end 80.01 80.01) (width 0.25) (layer "B.Cu") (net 23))
 (segment (start 101.6 72.39) (end 101.6 78.74) (width 0.25) (layer "B.Cu") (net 23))
 (segment (start 111.76 79.375) (end 106.68 84.455) (width 0.25) (layer "B.Cu") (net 24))
 (segment (start 113.03 70.49) (end 113.03 71.12) (width 0.25) (layer "B.Cu") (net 24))
 (segment (start 80.01 84.455) (end 77.47 81.915) (width 0.25) (layer "B.Cu") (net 24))
 (segment (start 77.47 81.915) (end 77.47 77.47) (width 0.25) (layer "B.Cu") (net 24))
 (segment (start 111.76 72.39) (end 111.76 79.375) (width 0.25) (layer "B.Cu") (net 24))
 (segment (start 113.03 71.12) (end 111.76 72.39) (width 0.25) (layer "B.Cu") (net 24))
 (segment (start 106.68 84.455) (end 80.01 84.455) (width 0.25) (layer "B.Cu") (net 24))
 (segment (start 75.565 74.93) (end 74.93 75.565) (width 0.25) (layer "B.Cu") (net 25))
 (segment (start 88.9 74.93) (end 75.565 74.93) (width 0.25) (layer "B.Cu") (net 25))
 (segment (start 90.17 71.12) (end 91.44 72.39) (width 0.25) (layer "B.Cu") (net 25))
 (segment (start 90.17 70.49) (end 90.17 71.12) (width 0.25) (layer "B.Cu") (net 25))
 (segment (start 74.93 75.565) (end 74.93 77.47) (width 0.25) (layer "B.Cu") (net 25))
 (segment (start 91.44 72.39) (end 88.9 74.93) (width 0.25) (layer "B.Cu") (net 25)))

